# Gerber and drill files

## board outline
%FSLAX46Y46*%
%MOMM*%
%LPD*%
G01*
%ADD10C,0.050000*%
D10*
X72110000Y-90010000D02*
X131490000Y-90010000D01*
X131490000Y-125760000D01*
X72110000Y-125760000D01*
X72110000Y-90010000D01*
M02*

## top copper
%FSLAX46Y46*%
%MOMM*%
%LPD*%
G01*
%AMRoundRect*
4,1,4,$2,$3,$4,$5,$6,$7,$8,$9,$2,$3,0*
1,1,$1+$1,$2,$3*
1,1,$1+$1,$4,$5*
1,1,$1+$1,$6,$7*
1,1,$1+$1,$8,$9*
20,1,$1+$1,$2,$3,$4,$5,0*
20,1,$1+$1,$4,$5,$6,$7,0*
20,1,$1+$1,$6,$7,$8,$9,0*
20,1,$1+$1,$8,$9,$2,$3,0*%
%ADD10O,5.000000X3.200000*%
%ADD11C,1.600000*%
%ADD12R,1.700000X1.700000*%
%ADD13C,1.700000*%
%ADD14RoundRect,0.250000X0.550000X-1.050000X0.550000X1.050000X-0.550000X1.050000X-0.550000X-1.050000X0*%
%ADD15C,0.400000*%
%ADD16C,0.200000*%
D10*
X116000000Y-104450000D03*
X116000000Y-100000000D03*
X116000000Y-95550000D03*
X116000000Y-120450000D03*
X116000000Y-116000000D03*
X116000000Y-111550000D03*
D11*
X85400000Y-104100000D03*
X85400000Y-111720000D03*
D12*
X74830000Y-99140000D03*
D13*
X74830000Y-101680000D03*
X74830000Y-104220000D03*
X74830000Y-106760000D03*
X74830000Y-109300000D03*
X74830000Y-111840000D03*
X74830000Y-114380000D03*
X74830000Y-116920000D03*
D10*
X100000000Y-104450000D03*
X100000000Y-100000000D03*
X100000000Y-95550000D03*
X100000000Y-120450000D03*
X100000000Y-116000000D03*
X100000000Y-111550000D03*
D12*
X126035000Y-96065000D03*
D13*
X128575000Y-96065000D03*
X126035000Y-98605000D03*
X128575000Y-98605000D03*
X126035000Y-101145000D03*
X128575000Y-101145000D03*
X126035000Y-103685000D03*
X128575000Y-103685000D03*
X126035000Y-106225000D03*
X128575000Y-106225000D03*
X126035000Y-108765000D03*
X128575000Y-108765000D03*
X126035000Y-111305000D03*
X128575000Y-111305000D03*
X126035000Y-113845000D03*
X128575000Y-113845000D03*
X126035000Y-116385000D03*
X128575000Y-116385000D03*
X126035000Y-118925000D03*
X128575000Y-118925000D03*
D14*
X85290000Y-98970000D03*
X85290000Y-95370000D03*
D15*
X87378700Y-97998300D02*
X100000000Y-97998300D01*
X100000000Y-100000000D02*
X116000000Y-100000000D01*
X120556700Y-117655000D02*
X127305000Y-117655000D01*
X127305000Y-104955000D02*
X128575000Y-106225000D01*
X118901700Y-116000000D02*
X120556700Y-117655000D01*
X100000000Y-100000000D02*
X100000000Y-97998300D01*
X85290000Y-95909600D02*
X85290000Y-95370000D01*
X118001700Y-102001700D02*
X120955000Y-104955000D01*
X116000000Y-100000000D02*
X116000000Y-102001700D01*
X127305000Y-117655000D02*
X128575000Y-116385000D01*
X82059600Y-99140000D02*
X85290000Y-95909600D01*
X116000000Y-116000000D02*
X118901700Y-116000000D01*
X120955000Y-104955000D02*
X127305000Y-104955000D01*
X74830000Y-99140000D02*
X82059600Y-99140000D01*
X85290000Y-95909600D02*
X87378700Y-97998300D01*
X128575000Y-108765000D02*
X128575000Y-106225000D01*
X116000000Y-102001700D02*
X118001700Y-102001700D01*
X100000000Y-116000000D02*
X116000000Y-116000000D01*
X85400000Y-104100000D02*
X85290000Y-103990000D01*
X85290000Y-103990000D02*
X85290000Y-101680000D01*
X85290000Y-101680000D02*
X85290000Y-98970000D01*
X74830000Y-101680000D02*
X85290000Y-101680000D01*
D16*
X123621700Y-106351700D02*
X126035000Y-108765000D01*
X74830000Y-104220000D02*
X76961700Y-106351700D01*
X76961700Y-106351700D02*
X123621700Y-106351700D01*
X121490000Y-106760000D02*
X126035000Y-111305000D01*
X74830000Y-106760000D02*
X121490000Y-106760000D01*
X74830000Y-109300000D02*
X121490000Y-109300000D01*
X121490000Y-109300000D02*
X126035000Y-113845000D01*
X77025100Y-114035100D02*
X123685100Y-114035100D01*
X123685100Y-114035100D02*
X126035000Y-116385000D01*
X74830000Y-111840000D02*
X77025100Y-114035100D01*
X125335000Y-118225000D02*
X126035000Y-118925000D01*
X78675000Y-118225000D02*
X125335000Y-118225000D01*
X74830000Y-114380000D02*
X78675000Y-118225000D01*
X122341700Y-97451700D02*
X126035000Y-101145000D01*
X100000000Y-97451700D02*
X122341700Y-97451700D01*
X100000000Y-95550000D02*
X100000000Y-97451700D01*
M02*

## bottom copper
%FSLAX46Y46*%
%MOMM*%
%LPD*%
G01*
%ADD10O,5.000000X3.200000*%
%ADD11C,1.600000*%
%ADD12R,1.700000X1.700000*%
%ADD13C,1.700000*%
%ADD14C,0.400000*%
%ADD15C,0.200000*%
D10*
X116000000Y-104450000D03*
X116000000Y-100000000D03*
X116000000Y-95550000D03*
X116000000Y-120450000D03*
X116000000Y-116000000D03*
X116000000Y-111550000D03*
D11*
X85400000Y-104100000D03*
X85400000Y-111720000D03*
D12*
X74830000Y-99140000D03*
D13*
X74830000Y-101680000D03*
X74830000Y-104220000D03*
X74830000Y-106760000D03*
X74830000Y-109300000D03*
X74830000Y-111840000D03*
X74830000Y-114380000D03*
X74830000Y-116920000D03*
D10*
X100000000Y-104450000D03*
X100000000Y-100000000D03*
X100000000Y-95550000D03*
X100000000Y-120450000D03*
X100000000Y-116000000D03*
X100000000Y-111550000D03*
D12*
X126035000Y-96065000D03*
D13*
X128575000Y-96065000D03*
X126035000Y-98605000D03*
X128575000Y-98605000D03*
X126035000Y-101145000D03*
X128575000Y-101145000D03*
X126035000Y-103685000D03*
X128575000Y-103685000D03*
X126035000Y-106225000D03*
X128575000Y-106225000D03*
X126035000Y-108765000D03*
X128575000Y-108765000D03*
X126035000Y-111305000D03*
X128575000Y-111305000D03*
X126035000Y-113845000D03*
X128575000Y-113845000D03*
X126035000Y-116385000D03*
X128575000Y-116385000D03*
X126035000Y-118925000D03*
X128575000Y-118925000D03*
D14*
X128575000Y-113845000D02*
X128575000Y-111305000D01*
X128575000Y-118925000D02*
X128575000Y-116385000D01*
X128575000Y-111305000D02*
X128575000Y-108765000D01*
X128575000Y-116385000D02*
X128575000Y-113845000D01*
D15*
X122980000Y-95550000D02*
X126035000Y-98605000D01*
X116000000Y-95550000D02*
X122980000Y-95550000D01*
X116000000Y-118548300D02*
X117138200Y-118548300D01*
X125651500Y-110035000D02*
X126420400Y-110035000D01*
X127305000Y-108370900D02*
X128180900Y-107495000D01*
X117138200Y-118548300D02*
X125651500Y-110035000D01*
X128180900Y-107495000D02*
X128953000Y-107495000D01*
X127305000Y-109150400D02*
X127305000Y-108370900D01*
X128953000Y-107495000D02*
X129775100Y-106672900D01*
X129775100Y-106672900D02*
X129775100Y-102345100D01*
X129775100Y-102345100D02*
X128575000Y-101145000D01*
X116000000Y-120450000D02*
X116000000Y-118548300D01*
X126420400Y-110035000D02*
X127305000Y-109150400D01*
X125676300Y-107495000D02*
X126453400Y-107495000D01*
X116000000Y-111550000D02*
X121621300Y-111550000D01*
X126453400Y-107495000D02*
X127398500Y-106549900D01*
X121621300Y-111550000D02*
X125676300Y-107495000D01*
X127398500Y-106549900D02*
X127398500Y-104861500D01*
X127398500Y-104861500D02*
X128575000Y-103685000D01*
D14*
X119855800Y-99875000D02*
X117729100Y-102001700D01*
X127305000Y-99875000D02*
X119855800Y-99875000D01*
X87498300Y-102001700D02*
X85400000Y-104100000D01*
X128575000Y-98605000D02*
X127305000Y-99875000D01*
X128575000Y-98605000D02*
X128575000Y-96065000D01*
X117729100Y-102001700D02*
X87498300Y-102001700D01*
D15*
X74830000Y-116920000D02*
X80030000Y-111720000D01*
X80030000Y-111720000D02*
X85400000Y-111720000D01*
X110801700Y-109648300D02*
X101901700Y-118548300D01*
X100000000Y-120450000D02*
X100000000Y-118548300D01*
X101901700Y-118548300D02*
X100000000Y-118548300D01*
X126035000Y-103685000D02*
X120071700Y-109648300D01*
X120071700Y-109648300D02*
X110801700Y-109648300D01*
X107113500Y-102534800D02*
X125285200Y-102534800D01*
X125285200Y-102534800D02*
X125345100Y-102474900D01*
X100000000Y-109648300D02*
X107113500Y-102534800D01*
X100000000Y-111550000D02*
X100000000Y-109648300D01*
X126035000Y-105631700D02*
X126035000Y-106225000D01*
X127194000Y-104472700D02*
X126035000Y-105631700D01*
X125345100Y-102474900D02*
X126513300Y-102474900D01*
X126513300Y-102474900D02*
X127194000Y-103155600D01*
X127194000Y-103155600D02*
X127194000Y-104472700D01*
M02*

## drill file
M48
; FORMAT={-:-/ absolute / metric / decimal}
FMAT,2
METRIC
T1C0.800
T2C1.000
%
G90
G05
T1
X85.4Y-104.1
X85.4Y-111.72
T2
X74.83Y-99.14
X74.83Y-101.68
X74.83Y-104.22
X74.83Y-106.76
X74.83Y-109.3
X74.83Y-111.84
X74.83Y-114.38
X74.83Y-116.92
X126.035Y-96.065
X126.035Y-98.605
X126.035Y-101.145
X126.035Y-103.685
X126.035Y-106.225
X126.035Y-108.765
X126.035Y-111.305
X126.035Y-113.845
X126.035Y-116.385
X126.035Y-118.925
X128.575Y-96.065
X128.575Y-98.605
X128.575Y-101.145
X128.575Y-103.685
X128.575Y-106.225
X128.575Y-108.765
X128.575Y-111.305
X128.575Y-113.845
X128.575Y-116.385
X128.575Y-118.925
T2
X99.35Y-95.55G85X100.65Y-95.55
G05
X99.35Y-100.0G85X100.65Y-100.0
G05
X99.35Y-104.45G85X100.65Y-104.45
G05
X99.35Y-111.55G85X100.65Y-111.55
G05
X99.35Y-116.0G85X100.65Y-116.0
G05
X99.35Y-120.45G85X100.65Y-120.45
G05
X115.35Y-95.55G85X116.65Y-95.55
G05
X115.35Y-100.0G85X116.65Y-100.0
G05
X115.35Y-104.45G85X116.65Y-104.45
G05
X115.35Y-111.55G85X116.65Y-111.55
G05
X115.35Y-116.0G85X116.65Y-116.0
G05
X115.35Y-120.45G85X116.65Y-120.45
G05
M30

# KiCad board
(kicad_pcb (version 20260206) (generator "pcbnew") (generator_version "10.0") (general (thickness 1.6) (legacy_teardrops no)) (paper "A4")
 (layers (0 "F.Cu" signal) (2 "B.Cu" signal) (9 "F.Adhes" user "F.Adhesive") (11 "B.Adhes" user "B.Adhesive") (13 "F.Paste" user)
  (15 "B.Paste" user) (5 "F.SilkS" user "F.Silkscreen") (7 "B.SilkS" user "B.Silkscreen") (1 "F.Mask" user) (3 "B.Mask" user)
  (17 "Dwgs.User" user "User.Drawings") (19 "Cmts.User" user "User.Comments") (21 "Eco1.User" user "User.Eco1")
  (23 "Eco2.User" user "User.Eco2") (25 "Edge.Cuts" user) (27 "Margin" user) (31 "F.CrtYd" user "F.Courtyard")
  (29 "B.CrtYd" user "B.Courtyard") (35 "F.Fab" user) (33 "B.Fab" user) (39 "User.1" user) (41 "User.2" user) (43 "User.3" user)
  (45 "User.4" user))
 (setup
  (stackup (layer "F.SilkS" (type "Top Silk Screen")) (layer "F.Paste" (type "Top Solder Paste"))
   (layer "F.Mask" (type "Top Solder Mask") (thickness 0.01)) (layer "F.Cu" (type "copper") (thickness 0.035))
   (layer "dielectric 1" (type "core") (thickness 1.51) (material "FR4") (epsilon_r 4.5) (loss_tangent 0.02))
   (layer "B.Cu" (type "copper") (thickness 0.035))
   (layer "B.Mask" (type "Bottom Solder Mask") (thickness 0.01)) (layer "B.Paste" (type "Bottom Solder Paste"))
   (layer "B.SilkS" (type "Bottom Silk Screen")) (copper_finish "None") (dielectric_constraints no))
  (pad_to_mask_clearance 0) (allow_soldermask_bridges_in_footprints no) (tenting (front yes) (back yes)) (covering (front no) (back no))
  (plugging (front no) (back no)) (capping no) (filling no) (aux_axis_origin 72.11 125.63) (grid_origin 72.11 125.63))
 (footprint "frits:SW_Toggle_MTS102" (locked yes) (layer "F.Cu") (at 116 100 90)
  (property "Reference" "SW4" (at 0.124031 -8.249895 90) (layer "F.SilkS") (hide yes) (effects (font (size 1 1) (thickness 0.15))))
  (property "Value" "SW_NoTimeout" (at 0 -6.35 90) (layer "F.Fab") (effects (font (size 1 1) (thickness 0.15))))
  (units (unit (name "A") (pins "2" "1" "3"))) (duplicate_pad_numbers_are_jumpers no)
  (pad "1" thru_hole oval (at -4.45 0 90) (size 3.2 5) (drill oval 1 2.3) (layers "*.Cu") (remove_unused_layers no)
   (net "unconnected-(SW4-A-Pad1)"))
  (pad "2" thru_hole oval (at 0 0 90) (size 3.2 5) (drill oval 1 2.3) (layers "*.Cu") (remove_unused_layers no) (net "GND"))
  (pad "3" thru_hole oval (at 4.45 0 90) (size 3.2 5) (drill oval 1 2.3) (layers "*.Cu") (remove_unused_layers no) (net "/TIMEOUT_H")))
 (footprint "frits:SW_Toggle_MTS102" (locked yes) (layer "F.Cu") (at 116 116 90)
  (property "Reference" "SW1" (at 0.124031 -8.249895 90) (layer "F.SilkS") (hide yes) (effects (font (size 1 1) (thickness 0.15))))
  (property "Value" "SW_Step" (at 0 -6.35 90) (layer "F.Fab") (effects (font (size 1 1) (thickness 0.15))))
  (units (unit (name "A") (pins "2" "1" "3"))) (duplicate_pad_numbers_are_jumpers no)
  (pad "1" thru_hole oval (at -4.45 0 90) (size 3.2 5) (drill oval 1 2.3) (layers "*.Cu") (remove_unused_layers no) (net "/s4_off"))
  (pad "2" thru_hole oval (at 0 0 90) (size 3.2 5) (drill oval 1 2.3) (layers "*.Cu") (remove_unused_layers no) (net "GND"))
  (pad "3" thru_hole oval (at 4.45 0 90) (size 3.2 5) (drill oval 1 2.3) (layers "*.Cu") (remove_unused_layers no) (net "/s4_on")))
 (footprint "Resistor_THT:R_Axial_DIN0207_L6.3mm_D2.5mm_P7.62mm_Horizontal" (layer "F.Cu") (at 85.4 104.1 -90)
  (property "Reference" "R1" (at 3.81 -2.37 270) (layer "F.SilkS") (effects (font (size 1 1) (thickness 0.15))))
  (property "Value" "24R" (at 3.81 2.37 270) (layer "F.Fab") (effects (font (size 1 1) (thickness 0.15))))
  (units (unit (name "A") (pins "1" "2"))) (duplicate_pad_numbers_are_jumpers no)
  (pad "1" thru_hole circle (at 0 0 270) (size 1.6 1.6) (drill 0.8) (layers "*.Cu" "*.Mask") (remove_unused_layers no) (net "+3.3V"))
  (pad "2" thru_hole circle (at 7.62 0 270) (size 1.6 1.6) (drill 0.8) (layers "*.Cu" "*.Mask") (remove_unused_layers no) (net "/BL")))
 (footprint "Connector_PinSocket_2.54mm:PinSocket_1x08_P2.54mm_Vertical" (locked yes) (layer "F.Cu") (at 74.83 99.14)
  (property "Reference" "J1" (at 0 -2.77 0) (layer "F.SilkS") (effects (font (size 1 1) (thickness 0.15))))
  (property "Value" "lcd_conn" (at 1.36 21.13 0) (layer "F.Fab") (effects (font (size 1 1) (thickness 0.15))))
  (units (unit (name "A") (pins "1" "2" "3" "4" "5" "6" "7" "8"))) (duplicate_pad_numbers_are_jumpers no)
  (pad "1" thru_hole rect (at 0 0) (size 1.7 1.7) (drill 1) (layers "*.Cu" "*.Mask") (remove_unused_layers no) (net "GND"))
  (pad "2" thru_hole circle (at 0 2.54) (size 1.7 1.7) (drill 1) (layers "*.Cu" "*.Mask") (remove_unused_layers no) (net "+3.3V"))
  (pad "3" thru_hole circle (at 0 5.08) (size 1.7 1.7) (drill 1) (layers "*.Cu" "*.Mask") (remove_unused_layers no) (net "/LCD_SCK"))
  (pad "4" thru_hole circle (at 0 7.62) (size 1.7 1.7) (drill 1) (layers "*.Cu" "*.Mask") (remove_unused_layers no) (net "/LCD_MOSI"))
  (pad "5" thru_hole circle (at 0 10.16) (size 1.7 1.7) (drill 1) (layers "*.Cu" "*.Mask") (remove_unused_layers no) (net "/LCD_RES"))
  (pad "6" thru_hole circle (at 0 12.7) (size 1.7 1.7) (drill 1) (layers "*.Cu" "*.Mask") (remove_unused_layers no) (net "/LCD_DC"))
  (pad "7" thru_hole circle (at 0 15.24) (size 1.7 1.7) (drill 1) (layers "*.Cu" "*.Mask") (remove_unused_layers no) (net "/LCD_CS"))
  (pad "8" thru_hole circle (at 0 17.78) (size 1.7 1.7) (drill 1) (layers "*.Cu" "*.Mask") (remove_unused_layers no) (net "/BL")))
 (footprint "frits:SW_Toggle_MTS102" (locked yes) (layer "F.Cu") (at 100 100 90)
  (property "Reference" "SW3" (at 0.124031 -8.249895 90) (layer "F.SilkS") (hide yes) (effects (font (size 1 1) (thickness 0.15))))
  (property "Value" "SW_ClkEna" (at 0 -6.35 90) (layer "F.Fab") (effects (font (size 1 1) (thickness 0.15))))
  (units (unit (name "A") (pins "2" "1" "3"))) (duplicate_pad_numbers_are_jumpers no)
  (pad "1" thru_hole oval (at -4.45 0 90) (size 3.2 5) (drill oval 1 2.3) (layers "*.Cu") (remove_unused_layers no)
   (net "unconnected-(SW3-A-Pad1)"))
  (pad "2" thru_hole oval (at 0 0 90) (size 3.2 5) (drill oval 1 2.3) (layers "*.Cu") (remove_unused_layers no) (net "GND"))
  (pad "3" thru_hole oval (at 4.45 0 90) (size 3.2 5) (drill oval 1 2.3) (layers "*.Cu") (remove_unused_layers no) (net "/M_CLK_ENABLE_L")))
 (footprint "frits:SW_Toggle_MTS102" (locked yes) (layer "F.Cu") (at 100 116 90)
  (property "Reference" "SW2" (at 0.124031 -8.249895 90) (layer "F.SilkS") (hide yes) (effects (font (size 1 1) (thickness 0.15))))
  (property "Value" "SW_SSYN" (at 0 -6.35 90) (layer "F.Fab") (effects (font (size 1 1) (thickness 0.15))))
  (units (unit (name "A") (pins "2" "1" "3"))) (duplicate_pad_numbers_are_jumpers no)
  (pad "1" thru_hole oval (at -4.45 0 90) (size 3.2 5) (drill oval 1 2.3) (layers "*.Cu") (remove_unused_layers no) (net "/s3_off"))
  (pad "2" thru_hole oval (at 0 0 90) (size 3.2 5) (drill oval 1 2.3) (layers "*.Cu") (remove_unused_layers no) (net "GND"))
  (pad "3" thru_hole oval (at 4.45 0 90) (size 3.2 5) (drill oval 1 2.3) (layers "*.Cu") (remove_unused_layers no) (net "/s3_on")))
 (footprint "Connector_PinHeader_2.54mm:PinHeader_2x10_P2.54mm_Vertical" (layer "F.Cu") (at 126.035 96.065)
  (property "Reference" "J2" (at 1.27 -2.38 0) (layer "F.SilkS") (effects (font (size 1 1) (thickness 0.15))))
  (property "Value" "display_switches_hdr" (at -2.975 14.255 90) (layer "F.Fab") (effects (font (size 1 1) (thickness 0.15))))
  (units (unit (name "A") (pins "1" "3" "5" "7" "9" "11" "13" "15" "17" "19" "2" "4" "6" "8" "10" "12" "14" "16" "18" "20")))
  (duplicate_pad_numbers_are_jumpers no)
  (pad "1" thru_hole rect (at 0 0) (size 1.7 1.7) (drill 1) (layers "*.Cu" "*.Mask") (remove_unused_layers no) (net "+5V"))
  (pad "2" thru_hole circle (at 2.54 0) (size 1.7 1.7) (drill 1) (layers "*.Cu" "*.Mask") (remove_unused_layers no) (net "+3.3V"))
  (pad "3" thru_hole circle (at 0 2.54) (size 1.7 1.7) (drill 1) (layers "*.Cu" "*.Mask") (remove_unused_layers no) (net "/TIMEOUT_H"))
  (pad "4" thru_hole circle (at 2.54 2.54) (size 1.7 1.7) (drill 1) (layers "*.Cu" "*.Mask") (remove_unused_layers no) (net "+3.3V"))
  (pad "5" thru_hole circle (at 0 5.08) (size 1.7 1.7) (drill 1) (layers "*.Cu" "*.Mask") (remove_unused_layers no) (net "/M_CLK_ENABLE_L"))
  (pad "6" thru_hole circle (at 2.54 5.08) (size 1.7 1.7) (drill 1) (layers "*.Cu" "*.Mask") (remove_unused_layers no) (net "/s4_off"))
  (pad "7" thru_hole circle (at 0 7.62) (size 1.7 1.7) (drill 1) (layers "*.Cu" "*.Mask") (remove_unused_layers no) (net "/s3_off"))
  (pad "8" thru_hole circle (at 2.54 7.62) (size 1.7 1.7) (drill 1) (layers "*.Cu" "*.Mask") (remove_unused_layers no) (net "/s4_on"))
  (pad "9" thru_hole circle (at 0 10.16) (size 1.7 1.7) (drill 1) (layers "*.Cu" "*.Mask") (remove_unused_layers no) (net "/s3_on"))
  (pad "10" thru_hole circle (at 2.54 10.16) (size 1.7 1.7) (drill 1) (layers "*.Cu" "*.Mask") (remove_unused_layers no) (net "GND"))
  (pad "11" thru_hole circle (at 0 12.7) (size 1.7 1.7) (drill 1) (layers "*.Cu" "*.Mask") (remove_unused_layers no) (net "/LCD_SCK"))
  (pad "12" thru_hole circle (at 2.54 12.7) (size 1.7 1.7) (drill 1) (layers "*.Cu" "*.Mask") (remove_unused_layers no) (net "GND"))
  (pad "13" thru_hole circle (at 0 15.24) (size 1.7 1.7) (drill 1) (layers "*.Cu" "*.Mask") (remove_unused_layers no) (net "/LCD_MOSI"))
  (pad "14" thru_hole circle (at 2.54 15.24) (size 1.7 1.7) (drill 1) (layers "*.Cu" "*.Mask") (remove_unused_layers no) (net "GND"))
  (pad "15" thru_hole circle (at 0 17.78) (size 1.7 1.7) (drill 1) (layers "*.Cu" "*.Mask") (remove_unused_layers no) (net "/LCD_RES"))
  (pad "16" thru_hole circle (at 2.54 17.78) (size 1.7 1.7) (drill 1) (layers "*.Cu" "*.Mask") (remove_unused_layers no) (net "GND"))
  (pad "17" thru_hole circle (at 0 20.32) (size 1.7 1.7) (drill 1) (layers "*.Cu" "*.Mask") (remove_unused_layers no) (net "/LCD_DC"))
  (pad "18" thru_hole circle (at 2.54 20.32) (size 1.7 1.7) (drill 1) (layers "*.Cu" "*.Mask") (remove_unused_layers no) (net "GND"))
  (pad "19" thru_hole circle (at 0 22.86) (size 1.7 1.7) (drill 1) (layers "*.Cu" "*.Mask") (remove_unused_layers no) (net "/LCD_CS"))
  (pad "20" thru_hole circle (at 2.54 22.86) (size 1.7 1.7) (drill 1) (layers "*.Cu" "*.Mask") (remove_unused_layers no) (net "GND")))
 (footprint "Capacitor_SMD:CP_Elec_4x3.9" (layer "F.Cu") (at 85.29 97.17 90)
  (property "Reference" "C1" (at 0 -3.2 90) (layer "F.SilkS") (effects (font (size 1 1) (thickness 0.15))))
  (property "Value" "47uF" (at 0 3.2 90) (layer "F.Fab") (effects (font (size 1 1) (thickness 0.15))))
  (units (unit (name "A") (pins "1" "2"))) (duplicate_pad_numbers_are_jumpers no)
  (pad "1" smd roundrect (at -1.8 0 90) (size 2.6 1.6) (layers "F.Cu" "F.Mask" "F.Paste") (roundrect_rratio 0.15625) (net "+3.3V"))
  (pad "2" smd roundrect (at 1.8 0 90) (size 2.6 1.6) (layers "F.Cu" "F.Mask" "F.Paste") (roundrect_rratio 0.15625) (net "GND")))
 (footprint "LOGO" (layer "B.Cu") (at 86.115939 107.717479 180)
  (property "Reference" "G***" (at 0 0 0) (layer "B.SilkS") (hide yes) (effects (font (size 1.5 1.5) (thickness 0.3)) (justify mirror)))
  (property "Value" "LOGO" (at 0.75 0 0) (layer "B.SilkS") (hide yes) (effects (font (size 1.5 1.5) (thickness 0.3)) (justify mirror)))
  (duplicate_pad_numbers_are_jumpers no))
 (gr_rect (start 72.11 90.01) (end 131.49 125.76) (stroke (width 0.05) (type default)) (fill no) (layer "Edge.Cuts"))
 (segment (start 87.3787 97.9983) (end 100 97.9983) (width 0.4) (layer "F.Cu") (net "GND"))
 (segment (start 100 100) (end 116 100) (width 0.4) (layer "F.Cu") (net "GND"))
 (segment (start 120.5567 117.655) (end 127.305 117.655) (width 0.4) (layer "F.Cu") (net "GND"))
 (segment (start 127.305 104.955) (end 128.575 106.225) (width 0.4) (layer "F.Cu") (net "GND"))
 (segment (start 118.9017 116) (end 120.5567 117.655) (width 0.4) (layer "F.Cu") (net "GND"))
 (segment (start 100 100) (end 100 97.9983) (width 0.4) (layer "F.Cu") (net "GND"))
 (segment (start 85.29 95.9096) (end 85.29 95.37) (width 0.4) (layer "F.Cu") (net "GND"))
 (segment (start 118.0017 102.0017) (end 120.955 104.955) (width 0.4) (layer "F.Cu") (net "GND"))
 (segment (start 116 100) (end 116 102.0017) (width 0.4) (layer "F.Cu") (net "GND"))
 (segment (start 127.305 117.655) (end 128.575 116.385) (width 0.4) (layer "F.Cu") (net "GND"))
 (segment (start 82.0596 99.14) (end 85.29 95.9096) (width 0.4) (layer "F.Cu") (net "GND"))
 (segment (start 116 116) (end 118.9017 116) (width 0.4) (layer "F.Cu") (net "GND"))
 (segment (start 120.955 104.955) (end 127.305 104.955) (width 0.4) (layer "F.Cu") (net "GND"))
 (segment (start 74.83 99.14) (end 82.0596 99.14) (width 0.4) (layer "F.Cu") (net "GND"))
 (segment (start 85.29 95.9096) (end 87.3787 97.9983) (width 0.4) (layer "F.Cu") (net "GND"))
 (segment (start 128.575 108.765) (end 128.575 106.225) (width 0.4) (layer "F.Cu") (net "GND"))
 (segment (start 116 102.0017) (end 118.0017 102.0017) (width 0.4) (layer "F.Cu") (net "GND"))
 (segment (start 100 116) (end 116 116) (width 0.4) (layer "F.Cu") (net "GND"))
 (segment (start 128.575 113.845) (end 128.575 111.305) (width 0.4) (layer "B.Cu") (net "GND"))
 (segment (start 128.575 118.925) (end 128.575 116.385) (width 0.4) (layer "B.Cu") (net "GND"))
 (segment (start 128.575 111.305) (end 128.575 108.765) (width 0.4) (layer "B.Cu") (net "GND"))
 (segment (start 128.575 116.385) (end 128.575 113.845) (width 0.4) (layer "B.Cu") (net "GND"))
 (segment (start 122.98 95.55) (end 126.035 98.605) (width 0.2) (layer "B.Cu") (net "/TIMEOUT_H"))
 (segment (start 116 95.55) (end 122.98 95.55) (width 0.2) (layer "B.Cu") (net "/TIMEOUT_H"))
 (segment (start 116 118.5483) (end 117.1382 118.5483) (width 0.2) (layer "B.Cu") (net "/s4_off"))
 (segment (start 125.6515 110.035) (end 126.4204 110.035) (width 0.2) (layer "B.Cu") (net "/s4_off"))
 (segment (start 127.305 108.3709) (end 128.1809 107.495) (width 0.2) (layer "B.Cu") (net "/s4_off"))
 (segment (start 117.1382 118.5483) (end 125.6515 110.035) (width 0.2) (layer "B.Cu") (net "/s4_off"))
 (segment (start 128.1809 107.495) (end 128.953 107.495) (width 0.2) (layer "B.Cu") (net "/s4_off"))
 (segment (start 127.305 109.1504) (end 127.305 108.3709) (width 0.2) (layer "B.Cu") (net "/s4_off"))
 (segment (start 128.953 107.495) (end 129.7751 106.6729) (width 0.2) (layer "B.Cu") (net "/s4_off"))
 (segment (start 129.7751 106.6729) (end 129.7751 102.3451) (width 0.2) (layer "B.Cu") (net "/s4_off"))
 (segment (start 129.7751 102.3451) (end 128.575 101.145) (width 0.2) (layer "B.Cu") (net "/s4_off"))
 (segment (start 116 120.45) (end 116 118.5483) (width 0.2) (layer "B.Cu") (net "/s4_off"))
 (segment (start 126.4204 110.035) (end 127.305 109.1504) (width 0.2) (layer "B.Cu") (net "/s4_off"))
 (segment (start 125.6763 107.495) (end 126.4534 107.495) (width 0.2) (layer "B.Cu") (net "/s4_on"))
 (segment (start 116 111.55) (end 121.6213 111.55) (width 0.2) (layer "B.Cu") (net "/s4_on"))
 (segment (start 126.4534 107.495) (end 127.3985 106.5499) (width 0.2) (layer "B.Cu") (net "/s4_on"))
 (segment (start 121.6213 111.55) (end 125.6763 107.495) (width 0.2) (layer "B.Cu") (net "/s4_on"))
 (segment (start 127.3985 106.5499) (end 127.3985 104.8615) (width 0.2) (layer "B.Cu") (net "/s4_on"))
 (segment (start 127.3985 104.8615) (end 128.575 103.685) (width 0.2) (layer "B.Cu") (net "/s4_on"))
 (segment (start 85.4 104.1) (end 85.29 103.99) (width 0.4) (layer "F.Cu") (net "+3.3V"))
 (segment (start 85.29 103.99) (end 85.29 101.68) (width 0.4) (layer "F.Cu") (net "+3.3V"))
 (segment (start 85.29 101.68) (end 85.29 98.97) (width 0.4) (layer "F.Cu") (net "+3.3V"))
 (segment (start 74.83 101.68) (end 85.29 101.68) (width 0.4) (layer "F.Cu") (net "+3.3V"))
 (segment (start 119.8558 99.875) (end 117.7291 102.0017) (width 0.4) (layer "B.Cu") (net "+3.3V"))
 (segment (start 127.305 99.875) (end 119.8558 99.875) (width 0.4) (layer "B.Cu") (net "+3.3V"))
 (segment (start 87.4983 102.0017) (end 85.4 104.1) (width 0.4) (layer "B.Cu") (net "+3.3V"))
 (segment (start 128.575 98.605) (end 127.305 99.875) (width 0.4) (layer "B.Cu") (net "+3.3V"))
 (segment (start 128.575 98.605) (end 128.575 96.065) (width 0.4) (layer "B.Cu") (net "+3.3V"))
 (segment (start 117.7291 102.0017) (end 87.4983 102.0017) (width 0.4) (layer "B.Cu") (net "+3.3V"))
 (segment (start 74.83 116.92) (end 80.03 111.72) (width 0.2) (layer "B.Cu") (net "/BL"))
 (segment (start 80.03 111.72) (end 85.4 111.72) (width 0.2) (layer "B.Cu") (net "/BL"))
 (segment (start 123.6217 106.3517) (end 126.035 108.765) (width 0.2) (layer "F.Cu") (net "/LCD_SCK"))
 (segment (start 74.83 104.22) (end 76.9617 106.3517) (width 0.2) (layer "F.Cu") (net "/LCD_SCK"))
 (segment (start 76.9617 106.3517) (end 123.6217 106.3517) (width 0.2) (layer "F.Cu") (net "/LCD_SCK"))
 (segment (start 121.49 106.76) (end 126.035 111.305) (width 0.2) (layer "F.Cu") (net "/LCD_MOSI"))
 (segment (start 74.83 106.76) (end 121.49 106.76) (width 0.2) (layer "F.Cu") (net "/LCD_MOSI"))
 (segment (start 74.83 109.3) (end 121.49 109.3) (width 0.2) (layer "F.Cu") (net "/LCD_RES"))
 (segment (start 121.49 109.3) (end 126.035 113.845) (width 0.2) (layer "F.Cu") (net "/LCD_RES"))
 (segment (start 77.0251 114.0351) (end 123.6851 114.0351) (width 0.2) (layer "F.Cu") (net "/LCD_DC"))
 (segment (start 123.6851 114.0351) (end 126.035 116.385) (width 0.2) (layer "F.Cu") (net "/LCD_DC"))
 (segment (start 74.83 111.84) (end 77.0251 114.0351) (width 0.2) (layer "F.Cu") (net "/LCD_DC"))
 (segment (start 125.335 118.225) (end 126.035 118.925) (width 0.2) (layer "F.Cu") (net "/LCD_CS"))
 (segment (start 78.675 118.225) (end 125.335 118.225) (width 0.2) (layer "F.Cu") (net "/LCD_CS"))
 (segment (start 74.83 114.38) (end 78.675 118.225) (width 0.2) (layer "F.Cu") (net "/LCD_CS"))
 (segment (start 122.3417 97.4517) (end 126.035 101.145) (width 0.2) (layer "F.Cu") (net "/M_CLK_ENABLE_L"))
 (segment (start 100 97.4517) (end 122.3417 97.4517) (width 0.2) (layer "F.Cu") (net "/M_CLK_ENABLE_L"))
 (segment (start 100 95.55) (end 100 97.4517) (width 0.2) (layer "F.Cu") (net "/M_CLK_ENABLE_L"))
 (segment (start 110.8017 109.6483) (end 101.9017 118.5483) (width 0.2) (layer "B.Cu") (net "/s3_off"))
 (segment (start 100 120.45) (end 100 118.5483) (width 0.2) (layer "B.Cu") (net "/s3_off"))
 (segment (start 101.9017 118.5483) (end 100 118.5483) (width 0.2) (layer "B.Cu") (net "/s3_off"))
 (segment (start 126.035 103.685) (end 120.0717 109.6483) (width 0.2) (layer "B.Cu") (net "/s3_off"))
 (segment (start 120.0717 109.6483) (end 110.8017 109.6483) (width 0.2) (layer "B.Cu") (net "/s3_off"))
 (segment (start 107.1135 102.5348) (end 125.2852 102.5348) (width 0.2) (layer "B.Cu") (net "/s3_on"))
 (segment (start 125.2852 102.5348) (end 125.3451 102.4749) (width 0.2) (layer "B.Cu") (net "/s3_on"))
 (segment (start 100 109.6483) (end 107.1135 102.5348) (width 0.2) (layer "B.Cu") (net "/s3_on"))
 (segment (start 100 111.55) (end 100 109.6483) (width 0.2) (layer "B.Cu") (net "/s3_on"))
 (segment (start 126.035 105.6317) (end 126.035 106.225) (width 0.2) (layer "B.Cu") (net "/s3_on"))
 (segment (start 127.194 104.4727) (end 126.035 105.6317) (width 0.2) (layer "B.Cu") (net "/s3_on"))
 (segment (start 125.3451 102.4749) (end 126.5133 102.4749) (width 0.2) (layer "B.Cu") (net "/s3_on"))
 (segment (start 126.5133 102.4749) (end 127.194 103.1556) (width 0.2) (layer "B.Cu") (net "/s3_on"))
 (segment (start 127.194 103.1556) (end 127.194 104.4727) (width 0.2) (layer "B.Cu") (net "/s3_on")))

